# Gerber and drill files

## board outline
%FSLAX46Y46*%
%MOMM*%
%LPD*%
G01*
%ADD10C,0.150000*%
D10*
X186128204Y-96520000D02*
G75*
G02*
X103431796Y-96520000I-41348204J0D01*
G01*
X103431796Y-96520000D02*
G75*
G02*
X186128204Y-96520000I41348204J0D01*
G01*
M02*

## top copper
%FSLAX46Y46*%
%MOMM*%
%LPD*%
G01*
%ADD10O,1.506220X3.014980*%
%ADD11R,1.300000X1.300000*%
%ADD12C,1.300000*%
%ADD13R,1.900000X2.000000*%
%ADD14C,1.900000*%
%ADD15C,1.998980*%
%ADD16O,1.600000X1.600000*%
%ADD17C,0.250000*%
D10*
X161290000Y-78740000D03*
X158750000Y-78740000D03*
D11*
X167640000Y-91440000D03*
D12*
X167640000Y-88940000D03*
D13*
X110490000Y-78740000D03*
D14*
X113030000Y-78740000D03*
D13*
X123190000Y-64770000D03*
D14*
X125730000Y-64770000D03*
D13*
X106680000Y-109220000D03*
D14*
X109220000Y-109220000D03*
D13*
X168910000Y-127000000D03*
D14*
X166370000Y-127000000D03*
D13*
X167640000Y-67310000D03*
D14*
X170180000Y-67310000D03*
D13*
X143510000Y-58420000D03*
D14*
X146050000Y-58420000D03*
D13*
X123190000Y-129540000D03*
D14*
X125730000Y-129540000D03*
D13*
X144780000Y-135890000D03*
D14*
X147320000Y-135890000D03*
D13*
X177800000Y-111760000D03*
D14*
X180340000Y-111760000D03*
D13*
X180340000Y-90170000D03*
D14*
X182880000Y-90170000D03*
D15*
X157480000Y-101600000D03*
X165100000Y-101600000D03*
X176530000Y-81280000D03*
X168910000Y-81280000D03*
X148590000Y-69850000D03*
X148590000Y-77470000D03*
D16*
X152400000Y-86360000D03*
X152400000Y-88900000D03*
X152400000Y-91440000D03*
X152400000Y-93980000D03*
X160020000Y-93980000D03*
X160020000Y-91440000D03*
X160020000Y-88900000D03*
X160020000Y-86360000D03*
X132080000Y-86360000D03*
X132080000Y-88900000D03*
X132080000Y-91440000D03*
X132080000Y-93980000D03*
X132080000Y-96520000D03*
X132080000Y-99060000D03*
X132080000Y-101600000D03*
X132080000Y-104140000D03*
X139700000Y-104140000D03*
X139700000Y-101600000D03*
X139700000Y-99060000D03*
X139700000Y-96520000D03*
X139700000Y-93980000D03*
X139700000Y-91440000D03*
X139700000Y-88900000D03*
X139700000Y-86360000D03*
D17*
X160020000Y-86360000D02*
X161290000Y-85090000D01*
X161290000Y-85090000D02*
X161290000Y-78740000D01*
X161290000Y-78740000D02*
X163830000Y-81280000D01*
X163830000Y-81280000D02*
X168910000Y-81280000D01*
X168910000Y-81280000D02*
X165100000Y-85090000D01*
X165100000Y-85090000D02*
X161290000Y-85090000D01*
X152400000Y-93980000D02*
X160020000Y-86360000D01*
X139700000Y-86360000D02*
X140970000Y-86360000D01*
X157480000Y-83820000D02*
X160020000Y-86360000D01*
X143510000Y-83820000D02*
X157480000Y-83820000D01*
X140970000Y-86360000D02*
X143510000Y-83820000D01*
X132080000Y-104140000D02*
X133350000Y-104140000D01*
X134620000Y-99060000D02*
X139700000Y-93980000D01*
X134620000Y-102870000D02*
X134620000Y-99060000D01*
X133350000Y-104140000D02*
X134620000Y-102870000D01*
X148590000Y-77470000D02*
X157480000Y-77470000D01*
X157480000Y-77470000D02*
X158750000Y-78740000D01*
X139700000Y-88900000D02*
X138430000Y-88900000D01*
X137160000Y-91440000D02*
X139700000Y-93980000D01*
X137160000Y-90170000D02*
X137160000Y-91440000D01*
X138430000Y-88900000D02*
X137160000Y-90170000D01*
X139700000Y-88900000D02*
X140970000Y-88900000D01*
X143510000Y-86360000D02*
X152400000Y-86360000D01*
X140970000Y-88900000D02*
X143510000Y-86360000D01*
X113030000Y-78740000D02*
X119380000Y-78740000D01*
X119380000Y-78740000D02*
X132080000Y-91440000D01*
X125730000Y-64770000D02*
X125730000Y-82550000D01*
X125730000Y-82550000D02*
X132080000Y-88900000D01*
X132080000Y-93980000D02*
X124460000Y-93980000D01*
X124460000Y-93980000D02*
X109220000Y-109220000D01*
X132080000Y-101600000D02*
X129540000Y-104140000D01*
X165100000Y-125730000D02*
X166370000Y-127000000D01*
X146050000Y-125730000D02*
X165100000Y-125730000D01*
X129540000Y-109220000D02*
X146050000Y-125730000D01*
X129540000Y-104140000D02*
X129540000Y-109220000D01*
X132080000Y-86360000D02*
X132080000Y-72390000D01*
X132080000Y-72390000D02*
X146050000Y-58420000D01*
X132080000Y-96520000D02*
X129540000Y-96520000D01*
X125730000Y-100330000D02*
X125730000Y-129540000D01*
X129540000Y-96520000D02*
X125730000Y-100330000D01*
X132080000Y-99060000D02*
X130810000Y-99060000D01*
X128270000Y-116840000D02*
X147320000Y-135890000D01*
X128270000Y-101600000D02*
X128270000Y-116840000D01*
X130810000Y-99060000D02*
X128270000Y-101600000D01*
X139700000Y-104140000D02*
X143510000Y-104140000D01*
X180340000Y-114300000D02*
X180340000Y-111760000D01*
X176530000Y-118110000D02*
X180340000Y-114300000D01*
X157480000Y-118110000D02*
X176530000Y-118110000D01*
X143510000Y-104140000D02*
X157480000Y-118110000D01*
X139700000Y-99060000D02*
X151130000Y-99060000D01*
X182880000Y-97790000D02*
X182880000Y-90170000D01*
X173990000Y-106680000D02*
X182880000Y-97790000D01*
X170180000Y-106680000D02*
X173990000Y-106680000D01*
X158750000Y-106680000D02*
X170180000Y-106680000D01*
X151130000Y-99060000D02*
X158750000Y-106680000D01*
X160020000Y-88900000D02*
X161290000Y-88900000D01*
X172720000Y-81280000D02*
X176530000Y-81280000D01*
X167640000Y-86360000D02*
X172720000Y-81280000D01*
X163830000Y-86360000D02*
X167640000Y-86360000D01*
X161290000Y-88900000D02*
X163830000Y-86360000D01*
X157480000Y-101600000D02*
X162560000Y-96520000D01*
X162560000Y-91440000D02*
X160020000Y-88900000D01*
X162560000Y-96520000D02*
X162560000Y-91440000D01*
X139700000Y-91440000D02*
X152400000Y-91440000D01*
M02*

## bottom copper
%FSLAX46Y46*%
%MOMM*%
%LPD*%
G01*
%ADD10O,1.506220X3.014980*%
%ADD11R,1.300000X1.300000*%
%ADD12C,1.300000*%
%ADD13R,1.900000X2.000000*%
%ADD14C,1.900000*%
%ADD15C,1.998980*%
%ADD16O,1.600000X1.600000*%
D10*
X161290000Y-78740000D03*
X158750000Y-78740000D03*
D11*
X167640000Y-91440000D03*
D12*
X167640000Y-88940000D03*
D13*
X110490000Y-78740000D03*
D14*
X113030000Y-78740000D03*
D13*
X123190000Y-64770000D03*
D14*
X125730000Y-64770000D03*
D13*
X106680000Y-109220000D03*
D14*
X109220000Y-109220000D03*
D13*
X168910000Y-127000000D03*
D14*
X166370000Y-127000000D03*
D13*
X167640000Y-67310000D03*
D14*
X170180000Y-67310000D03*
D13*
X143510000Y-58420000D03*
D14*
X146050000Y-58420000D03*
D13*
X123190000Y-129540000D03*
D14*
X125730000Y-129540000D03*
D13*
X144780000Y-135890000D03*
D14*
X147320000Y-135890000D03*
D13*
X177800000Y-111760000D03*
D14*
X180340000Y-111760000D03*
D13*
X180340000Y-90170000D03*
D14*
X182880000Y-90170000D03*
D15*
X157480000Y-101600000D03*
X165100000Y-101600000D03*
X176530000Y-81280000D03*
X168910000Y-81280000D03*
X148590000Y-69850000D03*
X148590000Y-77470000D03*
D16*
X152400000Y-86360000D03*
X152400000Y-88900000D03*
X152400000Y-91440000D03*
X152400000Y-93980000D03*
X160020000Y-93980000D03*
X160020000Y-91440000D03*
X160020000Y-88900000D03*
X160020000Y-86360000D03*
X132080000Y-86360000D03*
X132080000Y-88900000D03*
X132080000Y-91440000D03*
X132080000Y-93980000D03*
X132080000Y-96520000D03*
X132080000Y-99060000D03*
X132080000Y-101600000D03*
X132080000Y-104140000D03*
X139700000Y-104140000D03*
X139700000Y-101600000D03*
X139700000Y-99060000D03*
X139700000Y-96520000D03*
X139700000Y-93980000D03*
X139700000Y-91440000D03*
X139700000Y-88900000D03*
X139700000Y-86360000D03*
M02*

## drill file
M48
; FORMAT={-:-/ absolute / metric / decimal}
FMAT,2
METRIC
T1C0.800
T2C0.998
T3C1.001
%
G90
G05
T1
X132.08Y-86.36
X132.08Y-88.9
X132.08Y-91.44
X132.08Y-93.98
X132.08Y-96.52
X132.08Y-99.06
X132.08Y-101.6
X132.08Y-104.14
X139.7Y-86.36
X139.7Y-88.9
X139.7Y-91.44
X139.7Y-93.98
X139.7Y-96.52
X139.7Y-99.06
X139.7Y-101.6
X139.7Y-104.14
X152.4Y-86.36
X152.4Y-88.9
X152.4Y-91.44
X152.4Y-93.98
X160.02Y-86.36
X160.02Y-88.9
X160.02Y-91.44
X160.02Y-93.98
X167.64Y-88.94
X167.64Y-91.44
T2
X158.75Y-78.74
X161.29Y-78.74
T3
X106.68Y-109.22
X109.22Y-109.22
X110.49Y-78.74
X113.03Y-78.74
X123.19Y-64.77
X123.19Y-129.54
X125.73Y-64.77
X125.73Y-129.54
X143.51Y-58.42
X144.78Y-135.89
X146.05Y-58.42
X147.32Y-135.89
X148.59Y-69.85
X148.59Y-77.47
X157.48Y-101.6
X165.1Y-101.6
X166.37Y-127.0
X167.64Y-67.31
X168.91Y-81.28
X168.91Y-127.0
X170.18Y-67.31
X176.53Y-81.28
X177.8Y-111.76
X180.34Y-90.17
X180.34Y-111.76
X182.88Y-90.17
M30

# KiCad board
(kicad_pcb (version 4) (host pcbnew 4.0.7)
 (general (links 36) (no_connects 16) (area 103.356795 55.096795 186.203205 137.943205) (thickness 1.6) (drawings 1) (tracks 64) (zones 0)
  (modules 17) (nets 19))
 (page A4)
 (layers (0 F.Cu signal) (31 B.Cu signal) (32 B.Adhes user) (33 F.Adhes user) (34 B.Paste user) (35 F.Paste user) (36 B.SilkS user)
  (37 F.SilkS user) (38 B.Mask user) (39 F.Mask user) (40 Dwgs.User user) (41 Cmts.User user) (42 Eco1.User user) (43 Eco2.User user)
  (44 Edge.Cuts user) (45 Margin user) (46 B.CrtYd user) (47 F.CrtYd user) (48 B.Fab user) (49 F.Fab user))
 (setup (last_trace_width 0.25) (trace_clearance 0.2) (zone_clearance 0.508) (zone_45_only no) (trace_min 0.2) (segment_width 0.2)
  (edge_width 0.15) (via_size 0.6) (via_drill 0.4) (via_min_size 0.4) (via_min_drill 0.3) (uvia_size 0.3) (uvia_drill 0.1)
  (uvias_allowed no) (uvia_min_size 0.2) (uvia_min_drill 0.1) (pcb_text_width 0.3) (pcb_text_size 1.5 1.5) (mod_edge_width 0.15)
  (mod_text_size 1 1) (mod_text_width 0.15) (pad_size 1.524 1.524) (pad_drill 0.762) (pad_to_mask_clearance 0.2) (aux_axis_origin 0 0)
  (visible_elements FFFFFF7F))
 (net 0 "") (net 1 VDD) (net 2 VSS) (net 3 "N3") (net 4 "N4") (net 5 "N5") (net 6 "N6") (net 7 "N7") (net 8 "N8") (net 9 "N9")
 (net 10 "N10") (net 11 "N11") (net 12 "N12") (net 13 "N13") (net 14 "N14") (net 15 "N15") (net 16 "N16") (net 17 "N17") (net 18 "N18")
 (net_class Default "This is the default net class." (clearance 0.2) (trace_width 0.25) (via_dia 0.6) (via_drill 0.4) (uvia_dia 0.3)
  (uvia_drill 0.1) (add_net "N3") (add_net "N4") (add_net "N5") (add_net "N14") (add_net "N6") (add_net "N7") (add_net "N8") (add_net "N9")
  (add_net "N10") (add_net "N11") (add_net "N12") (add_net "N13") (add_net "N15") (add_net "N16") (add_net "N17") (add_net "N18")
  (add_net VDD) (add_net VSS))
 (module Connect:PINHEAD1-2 (layer F.Cu) (at 160.02 78.74 180)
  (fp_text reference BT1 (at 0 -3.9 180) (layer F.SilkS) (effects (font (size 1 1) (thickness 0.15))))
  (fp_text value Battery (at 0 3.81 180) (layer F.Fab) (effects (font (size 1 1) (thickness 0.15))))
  (pad 1 thru_hole oval (at -1.27 0 180) (size 1.50622 3.01498) (drill 0.99822) (layers *.Cu *.Mask) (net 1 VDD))
  (pad 2 thru_hole oval (at 1.27 0 180) (size 1.50622 3.01498) (drill 0.99822) (layers *.Cu *.Mask) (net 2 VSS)))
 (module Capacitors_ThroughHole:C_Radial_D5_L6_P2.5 (layer F.Cu) (at 167.64 91.44 90)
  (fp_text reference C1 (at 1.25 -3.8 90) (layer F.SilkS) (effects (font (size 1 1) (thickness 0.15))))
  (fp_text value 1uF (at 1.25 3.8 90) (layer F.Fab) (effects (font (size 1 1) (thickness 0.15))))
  (pad 1 thru_hole rect (at 0 0 90) (size 1.3 1.3) (drill 0.8) (layers *.Cu *.Mask F.SilkS) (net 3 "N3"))
  (pad 2 thru_hole circle (at 2.5 0 90) (size 1.3 1.3) (drill 0.8) (layers *.Cu *.Mask F.SilkS) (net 2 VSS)))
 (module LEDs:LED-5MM (layer F.Cu) (at 110.49 78.74)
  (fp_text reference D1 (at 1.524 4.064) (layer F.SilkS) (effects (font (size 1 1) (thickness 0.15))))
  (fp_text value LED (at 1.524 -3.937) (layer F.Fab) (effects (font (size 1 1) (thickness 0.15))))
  (pad 1 thru_hole rect (at 0 0 90) (size 2 1.9) (drill 1.00076) (layers *.Cu *.Mask F.SilkS) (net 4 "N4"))
  (pad 2 thru_hole circle (at 2.54 0) (size 1.9 1.9) (drill 1.00076) (layers *.Cu *.Mask F.SilkS) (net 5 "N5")))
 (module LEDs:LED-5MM (layer F.Cu) (at 123.19 64.77)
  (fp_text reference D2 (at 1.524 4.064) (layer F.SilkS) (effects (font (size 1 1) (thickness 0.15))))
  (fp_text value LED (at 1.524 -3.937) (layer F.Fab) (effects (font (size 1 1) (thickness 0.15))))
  (pad 1 thru_hole rect (at 0 0 90) (size 2 1.9) (drill 1.00076) (layers *.Cu *.Mask F.SilkS) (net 4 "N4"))
  (pad 2 thru_hole circle (at 2.54 0) (size 1.9 1.9) (drill 1.00076) (layers *.Cu *.Mask F.SilkS) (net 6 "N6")))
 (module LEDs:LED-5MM (layer F.Cu) (at 106.68 109.22)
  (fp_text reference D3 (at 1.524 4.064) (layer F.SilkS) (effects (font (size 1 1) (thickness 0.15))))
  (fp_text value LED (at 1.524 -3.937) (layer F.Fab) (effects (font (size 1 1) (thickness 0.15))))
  (pad 1 thru_hole rect (at 0 0 90) (size 2 1.9) (drill 1.00076) (layers *.Cu *.Mask F.SilkS) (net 4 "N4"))
  (pad 2 thru_hole circle (at 2.54 0) (size 1.9 1.9) (drill 1.00076) (layers *.Cu *.Mask F.SilkS) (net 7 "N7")))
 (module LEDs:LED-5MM (layer F.Cu) (at 168.91 127 180)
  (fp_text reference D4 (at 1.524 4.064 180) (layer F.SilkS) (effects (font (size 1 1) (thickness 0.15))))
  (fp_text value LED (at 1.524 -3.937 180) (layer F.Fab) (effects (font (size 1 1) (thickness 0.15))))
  (pad 1 thru_hole rect (at 0 0 270) (size 2 1.9) (drill 1.00076) (layers *.Cu *.Mask F.SilkS) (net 4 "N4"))
  (pad 2 thru_hole circle (at 2.54 0 180) (size 1.9 1.9) (drill 1.00076) (layers *.Cu *.Mask F.SilkS) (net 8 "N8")))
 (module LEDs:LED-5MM (layer F.Cu) (at 167.64 67.31)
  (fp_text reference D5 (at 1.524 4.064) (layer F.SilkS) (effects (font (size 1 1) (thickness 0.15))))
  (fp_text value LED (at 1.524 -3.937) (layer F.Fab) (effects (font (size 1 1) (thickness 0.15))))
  (pad 1 thru_hole rect (at 0 0 90) (size 2 1.9) (drill 1.00076) (layers *.Cu *.Mask F.SilkS) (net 4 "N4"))
  (pad 2 thru_hole circle (at 2.54 0) (size 1.9 1.9) (drill 1.00076) (layers *.Cu *.Mask F.SilkS) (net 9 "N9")))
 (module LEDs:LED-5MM (layer F.Cu) (at 143.51 58.42)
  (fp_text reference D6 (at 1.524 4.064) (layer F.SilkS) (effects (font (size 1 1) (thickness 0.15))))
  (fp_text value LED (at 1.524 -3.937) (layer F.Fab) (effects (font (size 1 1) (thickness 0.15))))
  (pad 1 thru_hole rect (at 0 0 90) (size 2 1.9) (drill 1.00076) (layers *.Cu *.Mask F.SilkS) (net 4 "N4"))
  (pad 2 thru_hole circle (at 2.54 0) (size 1.9 1.9) (drill 1.00076) (layers *.Cu *.Mask F.SilkS) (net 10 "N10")))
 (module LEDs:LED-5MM (layer F.Cu) (at 123.19 129.54)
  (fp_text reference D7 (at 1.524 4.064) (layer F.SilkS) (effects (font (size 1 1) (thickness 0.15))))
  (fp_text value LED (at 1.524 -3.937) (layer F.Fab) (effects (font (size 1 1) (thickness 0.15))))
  (pad 1 thru_hole rect (at 0 0 90) (size 2 1.9) (drill 1.00076) (layers *.Cu *.Mask F.SilkS) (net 4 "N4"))
  (pad 2 thru_hole circle (at 2.54 0) (size 1.9 1.9) (drill 1.00076) (layers *.Cu *.Mask F.SilkS) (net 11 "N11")))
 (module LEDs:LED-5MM (layer F.Cu) (at 144.78 135.89)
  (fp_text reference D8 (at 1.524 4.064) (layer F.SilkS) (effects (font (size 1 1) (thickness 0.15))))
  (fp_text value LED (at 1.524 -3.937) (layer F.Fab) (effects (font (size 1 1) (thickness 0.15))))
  (pad 1 thru_hole rect (at 0 0 90) (size 2 1.9) (drill 1.00076) (layers *.Cu *.Mask F.SilkS) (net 4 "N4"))
  (pad 2 thru_hole circle (at 2.54 0) (size 1.9 1.9) (drill 1.00076) (layers *.Cu *.Mask F.SilkS) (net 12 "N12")))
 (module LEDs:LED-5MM (layer F.Cu) (at 177.8 111.76)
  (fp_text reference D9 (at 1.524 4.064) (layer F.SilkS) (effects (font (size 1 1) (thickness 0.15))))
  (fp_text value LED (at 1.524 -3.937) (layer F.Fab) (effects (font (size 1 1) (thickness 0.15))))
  (pad 1 thru_hole rect (at 0 0 90) (size 2 1.9) (drill 1.00076) (layers *.Cu *.Mask F.SilkS) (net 4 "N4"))
  (pad 2 thru_hole circle (at 2.54 0) (size 1.9 1.9) (drill 1.00076) (layers *.Cu *.Mask F.SilkS) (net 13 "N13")))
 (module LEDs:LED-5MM (layer F.Cu) (at 180.34 90.17)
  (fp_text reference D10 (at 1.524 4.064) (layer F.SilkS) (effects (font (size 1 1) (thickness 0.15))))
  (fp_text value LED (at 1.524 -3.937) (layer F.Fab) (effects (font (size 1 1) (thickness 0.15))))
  (pad 1 thru_hole rect (at 0 0 90) (size 2 1.9) (drill 1.00076) (layers *.Cu *.Mask F.SilkS) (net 4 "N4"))
  (pad 2 thru_hole circle (at 2.54 0) (size 1.9 1.9) (drill 1.00076) (layers *.Cu *.Mask F.SilkS) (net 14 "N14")))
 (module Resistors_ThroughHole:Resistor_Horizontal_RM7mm (layer F.Cu) (at 157.48 101.6)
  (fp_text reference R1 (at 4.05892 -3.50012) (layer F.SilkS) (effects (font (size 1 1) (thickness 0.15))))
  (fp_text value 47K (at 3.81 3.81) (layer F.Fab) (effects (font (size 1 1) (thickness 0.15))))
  (pad 1 thru_hole circle (at 0 0) (size 1.99898 1.99898) (drill 1.00076) (layers *.Cu *.SilkS *.Mask) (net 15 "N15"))
  (pad 2 thru_hole circle (at 7.62 0) (size 1.99898 1.99898) (drill 1.00076) (layers *.Cu *.SilkS *.Mask) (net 3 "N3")))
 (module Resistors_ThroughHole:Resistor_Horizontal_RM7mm (layer F.Cu) (at 176.53 81.28 180)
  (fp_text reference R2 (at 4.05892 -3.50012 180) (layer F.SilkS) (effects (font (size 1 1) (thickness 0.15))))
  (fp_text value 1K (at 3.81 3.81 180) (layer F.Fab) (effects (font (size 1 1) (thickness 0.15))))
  (pad 1 thru_hole circle (at 0 0 180) (size 1.99898 1.99898) (drill 1.00076) (layers *.Cu *.SilkS *.Mask) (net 15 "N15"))
  (pad 2 thru_hole circle (at 7.62 0 180) (size 1.99898 1.99898) (drill 1.00076) (layers *.Cu *.SilkS *.Mask) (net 1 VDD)))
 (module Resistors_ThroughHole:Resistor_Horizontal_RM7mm (layer F.Cu) (at 148.59 69.85 270)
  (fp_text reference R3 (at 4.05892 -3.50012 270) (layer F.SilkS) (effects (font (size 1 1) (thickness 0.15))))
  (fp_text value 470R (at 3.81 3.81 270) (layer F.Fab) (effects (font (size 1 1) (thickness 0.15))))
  (pad 1 thru_hole circle (at 0 0 270) (size 1.99898 1.99898) (drill 1.00076) (layers *.Cu *.SilkS *.Mask) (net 4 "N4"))
  (pad 2 thru_hole circle (at 7.62 0 270) (size 1.99898 1.99898) (drill 1.00076) (layers *.Cu *.SilkS *.Mask) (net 2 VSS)))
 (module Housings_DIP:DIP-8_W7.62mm (layer F.Cu) (at 152.4 86.36)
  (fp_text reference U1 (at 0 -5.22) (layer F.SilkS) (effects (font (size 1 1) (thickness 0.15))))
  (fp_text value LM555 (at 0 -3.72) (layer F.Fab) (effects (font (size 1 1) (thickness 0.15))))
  (pad 1 thru_hole oval (at 0 0) (size 1.6 1.6) (drill 0.8) (layers *.Cu *.Mask F.SilkS) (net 2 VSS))
  (pad 2 thru_hole oval (at 0 2.54) (size 1.6 1.6) (drill 0.8) (layers *.Cu *.Mask F.SilkS) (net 3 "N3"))
  (pad 3 thru_hole oval (at 0 5.08) (size 1.6 1.6) (drill 0.8) (layers *.Cu *.Mask F.SilkS) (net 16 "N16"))
  (pad 4 thru_hole oval (at 0 7.62) (size 1.6 1.6) (drill 0.8) (layers *.Cu *.Mask F.SilkS) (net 1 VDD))
  (pad 5 thru_hole oval (at 7.62 7.62) (size 1.6 1.6) (drill 0.8) (layers *.Cu *.Mask F.SilkS) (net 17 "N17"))
  (pad 6 thru_hole oval (at 7.62 5.08) (size 1.6 1.6) (drill 0.8) (layers *.Cu *.Mask F.SilkS) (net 3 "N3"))
  (pad 7 thru_hole oval (at 7.62 2.54) (size 1.6 1.6) (drill 0.8) (layers *.Cu *.Mask F.SilkS) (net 15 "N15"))
  (pad 8 thru_hole oval (at 7.62 0) (size 1.6 1.6) (drill 0.8) (layers *.Cu *.Mask F.SilkS) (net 1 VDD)))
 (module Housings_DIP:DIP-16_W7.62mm (layer F.Cu) (at 132.08 86.36)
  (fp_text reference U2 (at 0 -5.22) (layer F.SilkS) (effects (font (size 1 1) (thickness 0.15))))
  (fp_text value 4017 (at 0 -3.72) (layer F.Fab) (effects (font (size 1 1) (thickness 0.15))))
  (pad 1 thru_hole oval (at 0 0) (size 1.6 1.6) (drill 0.8) (layers *.Cu *.Mask F.SilkS) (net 10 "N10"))
  (pad 2 thru_hole oval (at 0 2.54) (size 1.6 1.6) (drill 0.8) (layers *.Cu *.Mask F.SilkS) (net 6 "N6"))
  (pad 3 thru_hole oval (at 0 5.08) (size 1.6 1.6) (drill 0.8) (layers *.Cu *.Mask F.SilkS) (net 5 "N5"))
  (pad 4 thru_hole oval (at 0 7.62) (size 1.6 1.6) (drill 0.8) (layers *.Cu *.Mask F.SilkS) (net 7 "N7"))
  (pad 5 thru_hole oval (at 0 10.16) (size 1.6 1.6) (drill 0.8) (layers *.Cu *.Mask F.SilkS) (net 11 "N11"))
  (pad 6 thru_hole oval (at 0 12.7) (size 1.6 1.6) (drill 0.8) (layers *.Cu *.Mask F.SilkS) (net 12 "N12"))
  (pad 7 thru_hole oval (at 0 15.24) (size 1.6 1.6) (drill 0.8) (layers *.Cu *.Mask F.SilkS) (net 8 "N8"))
  (pad 8 thru_hole oval (at 0 17.78) (size 1.6 1.6) (drill 0.8) (layers *.Cu *.Mask F.SilkS) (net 2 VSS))
  (pad 9 thru_hole oval (at 7.62 17.78) (size 1.6 1.6) (drill 0.8) (layers *.Cu *.Mask F.SilkS) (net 13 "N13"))
  (pad 10 thru_hole oval (at 7.62 15.24) (size 1.6 1.6) (drill 0.8) (layers *.Cu *.Mask F.SilkS) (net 9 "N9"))
  (pad 11 thru_hole oval (at 7.62 12.7) (size 1.6 1.6) (drill 0.8) (layers *.Cu *.Mask F.SilkS) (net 14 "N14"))
  (pad 12 thru_hole oval (at 7.62 10.16) (size 1.6 1.6) (drill 0.8) (layers *.Cu *.Mask F.SilkS) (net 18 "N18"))
  (pad 13 thru_hole oval (at 7.62 7.62) (size 1.6 1.6) (drill 0.8) (layers *.Cu *.Mask F.SilkS) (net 2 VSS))
  (pad 14 thru_hole oval (at 7.62 5.08) (size 1.6 1.6) (drill 0.8) (layers *.Cu *.Mask F.SilkS) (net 16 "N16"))
  (pad 15 thru_hole oval (at 7.62 2.54) (size 1.6 1.6) (drill 0.8) (layers *.Cu *.Mask F.SilkS) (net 2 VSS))
  (pad 16 thru_hole oval (at 7.62 0) (size 1.6 1.6) (drill 0.8) (layers *.Cu *.Mask F.SilkS) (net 1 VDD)))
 (gr_circle (center 144.78 96.52) (end 175.26 124.46) (layer Edge.Cuts) (width 0.15))
 (segment (start 160.02 86.36) (end 161.29 85.09) (width 0.25) (layer F.Cu) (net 1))
 (segment (start 161.29 85.09) (end 161.29 78.74) (width 0.25) (layer F.Cu) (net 1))
 (segment (start 161.29 78.74) (end 163.83 81.28) (width 0.25) (layer F.Cu) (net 1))
 (segment (start 163.83 81.28) (end 168.91 81.28) (width 0.25) (layer F.Cu) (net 1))
 (segment (start 168.91 81.28) (end 165.1 85.09) (width 0.25) (layer F.Cu) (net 1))
 (segment (start 165.1 85.09) (end 161.29 85.09) (width 0.25) (layer F.Cu) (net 1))
 (segment (start 152.4 93.98) (end 160.02 86.36) (width 0.25) (layer F.Cu) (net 1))
 (segment (start 139.7 86.36) (end 140.97 86.36) (width 0.25) (layer F.Cu) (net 1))
 (segment (start 157.48 83.82) (end 160.02 86.36) (width 0.25) (layer F.Cu) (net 1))
 (segment (start 143.51 83.82) (end 157.48 83.82) (width 0.25) (layer F.Cu) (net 1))
 (segment (start 140.97 86.36) (end 143.51 83.82) (width 0.25) (layer F.Cu) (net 1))
 (segment (start 132.08 104.14) (end 133.35 104.14) (width 0.25) (layer F.Cu) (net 2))
 (segment (start 134.62 99.06) (end 139.7 93.98) (width 0.25) (layer F.Cu) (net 2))
 (segment (start 134.62 102.87) (end 134.62 99.06) (width 0.25) (layer F.Cu) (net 2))
 (segment (start 133.35 104.14) (end 134.62 102.87) (width 0.25) (layer F.Cu) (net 2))
 (segment (start 148.59 77.47) (end 157.48 77.47) (width 0.25) (layer F.Cu) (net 2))
 (segment (start 157.48 77.47) (end 158.75 78.74) (width 0.25) (layer F.Cu) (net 2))
 (segment (start 139.7 88.9) (end 138.43 88.9) (width 0.25) (layer F.Cu) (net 2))
 (segment (start 137.16 91.44) (end 139.7 93.98) (width 0.25) (layer F.Cu) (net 2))
 (segment (start 137.16 90.17) (end 137.16 91.44) (width 0.25) (layer F.Cu) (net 2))
 (segment (start 138.43 88.9) (end 137.16 90.17) (width 0.25) (layer F.Cu) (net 2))
 (segment (start 139.7 88.9) (end 140.97 88.9) (width 0.25) (layer F.Cu) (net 2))
 (segment (start 143.51 86.36) (end 152.4 86.36) (width 0.25) (layer F.Cu) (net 2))
 (segment (start 140.97 88.9) (end 143.51 86.36) (width 0.25) (layer F.Cu) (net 2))
 (segment (start 113.03 78.74) (end 119.38 78.74) (width 0.25) (layer F.Cu) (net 5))
 (segment (start 119.38 78.74) (end 132.08 91.44) (width 0.25) (layer F.Cu) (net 5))
 (segment (start 125.73 64.77) (end 125.73 82.55) (width 0.25) (layer F.Cu) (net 6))
 (segment (start 125.73 82.55) (end 132.08 88.9) (width 0.25) (layer F.Cu) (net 6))
 (segment (start 132.08 93.98) (end 124.46 93.98) (width 0.25) (layer F.Cu) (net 7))
 (segment (start 124.46 93.98) (end 109.22 109.22) (width 0.25) (layer F.Cu) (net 7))
 (segment (start 132.08 101.6) (end 129.54 104.14) (width 0.25) (layer F.Cu) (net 8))
 (segment (start 165.1 125.73) (end 166.37 127) (width 0.25) (layer F.Cu) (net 8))
 (segment (start 146.05 125.73) (end 165.1 125.73) (width 0.25) (layer F.Cu) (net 8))
 (segment (start 129.54 109.22) (end 146.05 125.73) (width 0.25) (layer F.Cu) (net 8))
 (segment (start 129.54 104.14) (end 129.54 109.22) (width 0.25) (layer F.Cu) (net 8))
 (segment (start 132.08 86.36) (end 132.08 72.39) (width 0.25) (layer F.Cu) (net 10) (status 400000))
 (segment (start 132.08 72.39) (end 146.05 58.42) (width 0.25) (layer F.Cu) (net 10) (status 800000))
 (segment (start 132.08 96.52) (end 129.54 96.52) (width 0.25) (layer F.Cu) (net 11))
 (segment (start 125.73 100.33) (end 125.73 129.54) (width 0.25) (layer F.Cu) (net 11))
 (segment (start 129.54 96.52) (end 125.73 100.33) (width 0.25) (layer F.Cu) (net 11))
 (segment (start 132.08 99.06) (end 130.81 99.06) (width 0.25) (layer F.Cu) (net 12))
 (segment (start 128.27 116.84) (end 147.32 135.89) (width 0.25) (layer F.Cu) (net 12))
 (segment (start 128.27 101.6) (end 128.27 116.84) (width 0.25) (layer F.Cu) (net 12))
 (segment (start 130.81 99.06) (end 128.27 101.6) (width 0.25) (layer F.Cu) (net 12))
 (segment (start 139.7 104.14) (end 143.51 104.14) (width 0.25) (layer F.Cu) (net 13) (status 400000))
 (segment (start 180.34 114.3) (end 180.34 111.76) (width 0.25) (layer F.Cu) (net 13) (status 800000))
 (segment (start 176.53 118.11) (end 180.34 114.3) (width 0.25) (layer F.Cu) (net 13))
 (segment (start 157.48 118.11) (end 176.53 118.11) (width 0.25) (layer F.Cu) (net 13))
 (segment (start 143.51 104.14) (end 157.48 118.11) (width 0.25) (layer F.Cu) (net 13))
 (segment (start 139.7 99.06) (end 151.13 99.06) (width 0.25) (layer F.Cu) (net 14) (status 400000))
 (segment (start 182.88 97.79) (end 182.88 90.17) (width 0.25) (layer F.Cu) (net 14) (status 800000))
 (segment (start 173.99 106.68) (end 182.88 97.79) (width 0.25) (layer F.Cu) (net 14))
 (segment (start 170.18 106.68) (end 173.99 106.68) (width 0.25) (layer F.Cu) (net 14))
 (segment (start 158.75 106.68) (end 170.18 106.68) (width 0.25) (layer F.Cu) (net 14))
 (segment (start 151.13 99.06) (end 158.75 106.68) (width 0.25) (layer F.Cu) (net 14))
 (segment (start 160.02 88.9) (end 161.29 88.9) (width 0.25) (layer F.Cu) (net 15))
 (segment (start 172.72 81.28) (end 176.53 81.28) (width 0.25) (layer F.Cu) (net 15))
 (segment (start 167.64 86.36) (end 172.72 81.28) (width 0.25) (layer F.Cu) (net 15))
 (segment (start 163.83 86.36) (end 167.64 86.36) (width 0.25) (layer F.Cu) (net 15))
 (segment (start 161.29 88.9) (end 163.83 86.36) (width 0.25) (layer F.Cu) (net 15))
 (segment (start 157.48 101.6) (end 162.56 96.52) (width 0.25) (layer F.Cu) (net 15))
 (segment (start 162.56 91.44) (end 160.02 88.9) (width 0.25) (layer F.Cu) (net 15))
 (segment (start 162.56 96.52) (end 162.56 91.44) (width 0.25) (layer F.Cu) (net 15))
 (segment (start 139.7 91.44) (end 152.4 91.44) (width 0.25) (layer F.Cu) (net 16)))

